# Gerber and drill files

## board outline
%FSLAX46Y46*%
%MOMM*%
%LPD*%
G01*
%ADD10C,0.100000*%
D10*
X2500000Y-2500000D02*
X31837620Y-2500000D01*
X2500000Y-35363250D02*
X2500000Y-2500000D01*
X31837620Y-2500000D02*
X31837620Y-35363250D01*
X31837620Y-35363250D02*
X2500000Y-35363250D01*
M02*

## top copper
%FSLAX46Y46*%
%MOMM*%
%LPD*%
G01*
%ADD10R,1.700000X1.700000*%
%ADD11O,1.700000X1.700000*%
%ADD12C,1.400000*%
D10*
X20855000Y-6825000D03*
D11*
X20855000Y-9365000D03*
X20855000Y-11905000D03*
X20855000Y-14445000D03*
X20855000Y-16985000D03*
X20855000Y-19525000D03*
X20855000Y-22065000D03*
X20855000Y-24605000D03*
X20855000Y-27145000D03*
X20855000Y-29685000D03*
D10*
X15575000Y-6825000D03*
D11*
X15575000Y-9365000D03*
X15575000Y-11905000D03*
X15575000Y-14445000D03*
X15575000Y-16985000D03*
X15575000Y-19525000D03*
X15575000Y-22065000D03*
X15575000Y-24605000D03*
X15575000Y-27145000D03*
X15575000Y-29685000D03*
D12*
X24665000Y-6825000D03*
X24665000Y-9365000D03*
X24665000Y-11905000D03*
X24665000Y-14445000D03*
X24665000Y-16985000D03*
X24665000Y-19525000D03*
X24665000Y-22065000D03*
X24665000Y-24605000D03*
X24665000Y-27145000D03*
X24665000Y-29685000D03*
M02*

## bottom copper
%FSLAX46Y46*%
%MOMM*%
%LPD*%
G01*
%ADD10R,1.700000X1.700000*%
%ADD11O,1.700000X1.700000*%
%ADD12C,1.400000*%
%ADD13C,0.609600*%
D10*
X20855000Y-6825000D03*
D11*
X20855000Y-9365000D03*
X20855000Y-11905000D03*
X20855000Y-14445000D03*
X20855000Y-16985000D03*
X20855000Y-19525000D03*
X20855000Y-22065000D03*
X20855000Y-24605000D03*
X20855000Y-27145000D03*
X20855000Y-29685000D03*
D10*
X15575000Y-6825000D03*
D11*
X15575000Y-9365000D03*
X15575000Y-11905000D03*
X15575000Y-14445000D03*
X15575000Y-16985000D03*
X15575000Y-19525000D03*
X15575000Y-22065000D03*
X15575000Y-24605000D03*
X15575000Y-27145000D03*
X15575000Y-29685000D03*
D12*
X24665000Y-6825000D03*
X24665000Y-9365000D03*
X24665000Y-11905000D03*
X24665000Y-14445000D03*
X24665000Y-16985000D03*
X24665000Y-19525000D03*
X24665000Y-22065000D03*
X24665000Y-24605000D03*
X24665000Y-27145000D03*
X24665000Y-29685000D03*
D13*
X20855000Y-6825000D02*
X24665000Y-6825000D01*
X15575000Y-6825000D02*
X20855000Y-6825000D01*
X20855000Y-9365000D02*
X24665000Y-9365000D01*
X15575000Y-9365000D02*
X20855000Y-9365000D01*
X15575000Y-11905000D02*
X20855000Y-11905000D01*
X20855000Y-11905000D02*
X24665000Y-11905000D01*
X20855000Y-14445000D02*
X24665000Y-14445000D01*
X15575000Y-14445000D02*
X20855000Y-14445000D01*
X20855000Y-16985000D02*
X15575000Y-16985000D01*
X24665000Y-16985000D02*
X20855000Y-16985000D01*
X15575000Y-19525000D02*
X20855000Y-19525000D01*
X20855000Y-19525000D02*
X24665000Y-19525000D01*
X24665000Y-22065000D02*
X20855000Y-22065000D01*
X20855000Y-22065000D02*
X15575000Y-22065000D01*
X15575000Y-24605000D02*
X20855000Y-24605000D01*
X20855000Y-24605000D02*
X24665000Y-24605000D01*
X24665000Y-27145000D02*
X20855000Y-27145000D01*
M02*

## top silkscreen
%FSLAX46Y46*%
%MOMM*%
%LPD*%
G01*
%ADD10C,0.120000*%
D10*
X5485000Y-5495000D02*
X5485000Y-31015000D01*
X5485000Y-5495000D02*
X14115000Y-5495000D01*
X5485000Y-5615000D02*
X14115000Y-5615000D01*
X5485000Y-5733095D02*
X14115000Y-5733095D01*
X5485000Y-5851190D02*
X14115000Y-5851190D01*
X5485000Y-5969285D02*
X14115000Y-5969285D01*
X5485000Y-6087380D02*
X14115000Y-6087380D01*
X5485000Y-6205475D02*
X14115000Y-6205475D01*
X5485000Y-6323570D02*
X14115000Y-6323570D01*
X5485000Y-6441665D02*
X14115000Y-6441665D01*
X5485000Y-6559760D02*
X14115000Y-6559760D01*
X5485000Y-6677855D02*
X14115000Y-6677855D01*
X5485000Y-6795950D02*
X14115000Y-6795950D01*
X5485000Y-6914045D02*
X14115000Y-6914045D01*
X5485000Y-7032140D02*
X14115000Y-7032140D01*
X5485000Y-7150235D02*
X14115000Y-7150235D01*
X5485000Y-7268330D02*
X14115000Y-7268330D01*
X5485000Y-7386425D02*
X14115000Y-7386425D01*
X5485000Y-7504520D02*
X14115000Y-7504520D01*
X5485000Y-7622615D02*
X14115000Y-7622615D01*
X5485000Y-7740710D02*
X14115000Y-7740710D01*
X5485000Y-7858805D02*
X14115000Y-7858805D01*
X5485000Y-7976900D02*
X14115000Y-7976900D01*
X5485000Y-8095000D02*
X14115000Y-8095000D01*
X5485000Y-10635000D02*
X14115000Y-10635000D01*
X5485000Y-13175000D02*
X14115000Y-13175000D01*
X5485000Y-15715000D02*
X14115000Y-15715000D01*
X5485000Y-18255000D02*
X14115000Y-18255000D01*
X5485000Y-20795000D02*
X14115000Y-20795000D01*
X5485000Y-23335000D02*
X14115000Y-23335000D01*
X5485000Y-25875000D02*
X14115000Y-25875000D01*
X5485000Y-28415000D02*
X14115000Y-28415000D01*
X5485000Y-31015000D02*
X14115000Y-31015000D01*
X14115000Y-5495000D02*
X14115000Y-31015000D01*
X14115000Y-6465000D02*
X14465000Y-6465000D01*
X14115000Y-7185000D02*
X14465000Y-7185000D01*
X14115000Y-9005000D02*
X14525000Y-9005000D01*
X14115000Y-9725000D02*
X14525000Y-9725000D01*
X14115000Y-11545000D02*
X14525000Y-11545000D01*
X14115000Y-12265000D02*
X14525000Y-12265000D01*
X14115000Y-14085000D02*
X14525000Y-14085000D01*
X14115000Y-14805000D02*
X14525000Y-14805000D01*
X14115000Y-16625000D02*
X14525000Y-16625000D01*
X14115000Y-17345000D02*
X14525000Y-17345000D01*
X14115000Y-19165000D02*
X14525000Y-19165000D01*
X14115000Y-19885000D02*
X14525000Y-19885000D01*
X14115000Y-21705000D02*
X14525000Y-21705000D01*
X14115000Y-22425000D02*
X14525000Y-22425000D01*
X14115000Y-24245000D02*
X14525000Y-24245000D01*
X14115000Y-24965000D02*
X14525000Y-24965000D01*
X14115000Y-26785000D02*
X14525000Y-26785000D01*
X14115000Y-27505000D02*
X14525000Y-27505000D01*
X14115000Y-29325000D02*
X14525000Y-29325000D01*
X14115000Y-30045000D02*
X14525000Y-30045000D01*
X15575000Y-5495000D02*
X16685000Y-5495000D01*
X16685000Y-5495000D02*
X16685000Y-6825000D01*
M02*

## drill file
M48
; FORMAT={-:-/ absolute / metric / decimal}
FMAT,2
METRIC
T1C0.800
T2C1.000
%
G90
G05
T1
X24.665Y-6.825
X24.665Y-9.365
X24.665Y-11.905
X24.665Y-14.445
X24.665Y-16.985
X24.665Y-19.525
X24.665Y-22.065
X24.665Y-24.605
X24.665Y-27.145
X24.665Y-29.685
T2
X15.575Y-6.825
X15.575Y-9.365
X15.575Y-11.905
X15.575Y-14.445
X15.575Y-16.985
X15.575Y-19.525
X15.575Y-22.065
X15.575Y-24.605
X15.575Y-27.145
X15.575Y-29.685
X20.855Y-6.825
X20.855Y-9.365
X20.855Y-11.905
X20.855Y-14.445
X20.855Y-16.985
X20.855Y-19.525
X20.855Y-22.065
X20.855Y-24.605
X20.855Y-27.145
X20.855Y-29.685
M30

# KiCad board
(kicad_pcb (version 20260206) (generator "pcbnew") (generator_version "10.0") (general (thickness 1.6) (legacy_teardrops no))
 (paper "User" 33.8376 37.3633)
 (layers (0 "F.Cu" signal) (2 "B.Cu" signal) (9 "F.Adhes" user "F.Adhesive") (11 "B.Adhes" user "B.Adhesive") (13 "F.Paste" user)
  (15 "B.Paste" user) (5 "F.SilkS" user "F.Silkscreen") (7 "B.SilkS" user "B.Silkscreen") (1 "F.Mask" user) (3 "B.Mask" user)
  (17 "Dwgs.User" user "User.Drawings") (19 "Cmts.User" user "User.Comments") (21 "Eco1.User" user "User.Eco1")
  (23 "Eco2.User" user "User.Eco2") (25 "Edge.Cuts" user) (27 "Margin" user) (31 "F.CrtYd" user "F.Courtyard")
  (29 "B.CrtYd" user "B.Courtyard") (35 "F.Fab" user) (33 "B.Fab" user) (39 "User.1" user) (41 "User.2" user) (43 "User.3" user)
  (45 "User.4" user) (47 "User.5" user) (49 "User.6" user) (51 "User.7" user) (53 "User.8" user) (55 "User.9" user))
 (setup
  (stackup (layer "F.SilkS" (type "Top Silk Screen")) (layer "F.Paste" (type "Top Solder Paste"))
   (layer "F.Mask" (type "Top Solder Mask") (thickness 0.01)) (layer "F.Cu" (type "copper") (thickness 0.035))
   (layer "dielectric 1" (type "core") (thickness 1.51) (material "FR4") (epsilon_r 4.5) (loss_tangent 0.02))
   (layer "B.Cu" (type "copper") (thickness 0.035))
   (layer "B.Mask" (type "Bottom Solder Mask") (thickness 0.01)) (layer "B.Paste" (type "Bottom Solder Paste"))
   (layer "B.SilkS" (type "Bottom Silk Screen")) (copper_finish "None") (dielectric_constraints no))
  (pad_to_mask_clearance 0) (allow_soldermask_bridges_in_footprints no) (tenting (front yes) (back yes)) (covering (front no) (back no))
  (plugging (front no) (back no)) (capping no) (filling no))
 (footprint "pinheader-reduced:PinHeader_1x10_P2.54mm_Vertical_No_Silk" (layer "F.Cu") (at 20.855 6.825)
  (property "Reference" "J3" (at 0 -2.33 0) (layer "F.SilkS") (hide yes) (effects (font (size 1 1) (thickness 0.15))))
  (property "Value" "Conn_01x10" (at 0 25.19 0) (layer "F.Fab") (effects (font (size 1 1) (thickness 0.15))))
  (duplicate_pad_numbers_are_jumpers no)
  (pad "1" thru_hole rect (at 0 0) (size 1.7 1.7) (drill 1) (layers "*.Cu" "*.Mask") (remove_unused_layers no) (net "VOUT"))
  (pad "2" thru_hole oval (at 0 2.54) (size 1.7 1.7) (drill 1) (layers "*.Cu" "*.Mask") (remove_unused_layers no) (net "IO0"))
  (pad "3" thru_hole oval (at 0 5.08) (size 1.7 1.7) (drill 1) (layers "*.Cu" "*.Mask") (remove_unused_layers no) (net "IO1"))
  (pad "4" thru_hole oval (at 0 7.62) (size 1.7 1.7) (drill 1) (layers "*.Cu" "*.Mask") (remove_unused_layers no) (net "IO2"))
  (pad "5" thru_hole oval (at 0 10.16) (size 1.7 1.7) (drill 1) (layers "*.Cu" "*.Mask") (remove_unused_layers no) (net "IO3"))
  (pad "6" thru_hole oval (at 0 12.7) (size 1.7 1.7) (drill 1) (layers "*.Cu" "*.Mask") (remove_unused_layers no) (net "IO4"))
  (pad "7" thru_hole oval (at 0 15.24) (size 1.7 1.7) (drill 1) (layers "*.Cu" "*.Mask") (remove_unused_layers no) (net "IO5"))
  (pad "8" thru_hole oval (at 0 17.78) (size 1.7 1.7) (drill 1) (layers "*.Cu" "*.Mask") (remove_unused_layers no) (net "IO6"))
  (pad "9" thru_hole oval (at 0 20.32) (size 1.7 1.7) (drill 1) (layers "*.Cu" "*.Mask") (remove_unused_layers no) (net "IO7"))
  (pad "10" thru_hole oval (at 0 22.86) (size 1.7 1.7) (drill 1) (layers "*.Cu" "*.Mask") (remove_unused_layers no) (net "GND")))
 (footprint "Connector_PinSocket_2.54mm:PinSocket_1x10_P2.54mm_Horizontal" (layer "F.Cu") (at 15.575 6.825)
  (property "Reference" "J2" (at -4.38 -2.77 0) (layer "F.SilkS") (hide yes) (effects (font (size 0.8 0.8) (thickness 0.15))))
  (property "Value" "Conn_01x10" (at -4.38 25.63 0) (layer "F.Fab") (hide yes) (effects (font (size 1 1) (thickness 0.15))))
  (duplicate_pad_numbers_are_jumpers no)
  (fp_line (start -10.09 -1.33) (end -10.09 24.19) (stroke (width 0.12) (type solid)) (layer "F.SilkS"))
  (fp_line (start -10.09 -1.33) (end -1.46 -1.33) (stroke (width 0.12) (type solid)) (layer "F.SilkS"))
  (fp_line (start -10.09 -1.21) (end -1.46 -1.21) (stroke (width 0.12) (type solid)) (layer "F.SilkS"))
  (fp_line (start -10.09 -1.091905) (end -1.46 -1.091905) (stroke (width 0.12) (type solid)) (layer "F.SilkS"))
  (fp_line (start -10.09 -0.97381) (end -1.46 -0.97381) (stroke (width 0.12) (type solid)) (layer "F.SilkS"))
  (fp_line (start -10.09 -0.855715) (end -1.46 -0.855715) (stroke (width 0.12) (type solid)) (layer "F.SilkS"))
  (fp_line (start -10.09 -0.73762) (end -1.46 -0.73762) (stroke (width 0.12) (type solid)) (layer "F.SilkS"))
  (fp_line (start -10.09 -0.619525) (end -1.46 -0.619525) (stroke (width 0.12) (type solid)) (layer "F.SilkS"))
  (fp_line (start -10.09 -0.50143) (end -1.46 -0.50143) (stroke (width 0.12) (type solid)) (layer "F.SilkS"))
  (fp_line (start -10.09 -0.383335) (end -1.46 -0.383335) (stroke (width 0.12) (type solid)) (layer "F.SilkS"))
  (fp_line (start -10.09 -0.26524) (end -1.46 -0.26524) (stroke (width 0.12) (type solid)) (layer "F.SilkS"))
  (fp_line (start -10.09 -0.147145) (end -1.46 -0.147145) (stroke (width 0.12) (type solid)) (layer "F.SilkS"))
  (fp_line (start -10.09 -0.02905) (end -1.46 -0.02905) (stroke (width 0.12) (type solid)) (layer "F.SilkS"))
  (fp_line (start -10.09 0.089045) (end -1.46 0.089045) (stroke (width 0.12) (type solid)) (layer "F.SilkS"))
  (fp_line (start -10.09 0.20714) (end -1.46 0.20714) (stroke (width 0.12) (type solid)) (layer "F.SilkS"))
  (fp_line (start -10.09 0.325235) (end -1.46 0.325235) (stroke (width 0.12) (type solid)) (layer "F.SilkS"))
  (fp_line (start -10.09 0.44333) (end -1.46 0.44333) (stroke (width 0.12) (type solid)) (layer "F.SilkS"))
  (fp_line (start -10.09 0.561425) (end -1.46 0.561425) (stroke (width 0.12) (type solid)) (layer "F.SilkS"))
  (fp_line (start -10.09 0.67952) (end -1.46 0.67952) (stroke (width 0.12) (type solid)) (layer "F.SilkS"))
  (fp_line (start -10.09 0.797615) (end -1.46 0.797615) (stroke (width 0.12) (type solid)) (layer "F.SilkS"))
  (fp_line (start -10.09 0.91571) (end -1.46 0.91571) (stroke (width 0.12) (type solid)) (layer "F.SilkS"))
  (fp_line (start -10.09 1.033805) (end -1.46 1.033805) (stroke (width 0.12) (type solid)) (layer "F.SilkS"))
  (fp_line (start -10.09 1.1519) (end -1.46 1.1519) (stroke (width 0.12) (type solid)) (layer "F.SilkS"))
  (fp_line (start -10.09 1.27) (end -1.46 1.27) (stroke (width 0.12) (type solid)) (layer "F.SilkS"))
  (fp_line (start -10.09 3.81) (end -1.46 3.81) (stroke (width 0.12) (type solid)) (layer "F.SilkS"))
  (fp_line (start -10.09 6.35) (end -1.46 6.35) (stroke (width 0.12) (type solid)) (layer "F.SilkS"))
  (fp_line (start -10.09 8.89) (end -1.46 8.89) (stroke (width 0.12) (type solid)) (layer "F.SilkS"))
  (fp_line (start -10.09 11.43) (end -1.46 11.43) (stroke (width 0.12) (type solid)) (layer "F.SilkS"))
  (fp_line (start -10.09 13.97) (end -1.46 13.97) (stroke (width 0.12) (type solid)) (layer "F.SilkS"))
  (fp_line (start -10.09 16.51) (end -1.46 16.51) (stroke (width 0.12) (type solid)) (layer "F.SilkS"))
  (fp_line (start -10.09 19.05) (end -1.46 19.05) (stroke (width 0.12) (type solid)) (layer "F.SilkS"))
  (fp_line (start -10.09 21.59) (end -1.46 21.59) (stroke (width 0.12) (type solid)) (layer "F.SilkS"))
  (fp_line (start -10.09 24.19) (end -1.46 24.19) (stroke (width 0.12) (type solid)) (layer "F.SilkS"))
  (fp_line (start -1.46 -1.33) (end -1.46 24.19) (stroke (width 0.12) (type solid)) (layer "F.SilkS"))
  (fp_line (start -1.46 -0.36) (end -1.11 -0.36) (stroke (width 0.12) (type solid)) (layer "F.SilkS"))
  (fp_line (start -1.46 0.36) (end -1.11 0.36) (stroke (width 0.12) (type solid)) (layer "F.SilkS"))
  (fp_line (start -1.46 2.18) (end -1.05 2.18) (stroke (width 0.12) (type solid)) (layer "F.SilkS"))
  (fp_line (start -1.46 2.9) (end -1.05 2.9) (stroke (width 0.12) (type solid)) (layer "F.SilkS"))
  (fp_line (start -1.46 4.72) (end -1.05 4.72) (stroke (width 0.12) (type solid)) (layer "F.SilkS"))
  (fp_line (start -1.46 5.44) (end -1.05 5.44) (stroke (width 0.12) (type solid)) (layer "F.SilkS"))
  (fp_line (start -1.46 7.26) (end -1.05 7.26) (stroke (width 0.12) (type solid)) (layer "F.SilkS"))
  (fp_line (start -1.46 7.98) (end -1.05 7.98) (stroke (width 0.12) (type solid)) (layer "F.SilkS"))
  (fp_line (start -1.46 9.8) (end -1.05 9.8) (stroke (width 0.12) (type solid)) (layer "F.SilkS"))
  (fp_line (start -1.46 10.52) (end -1.05 10.52) (stroke (width 0.12) (type solid)) (layer "F.SilkS"))
  (fp_line (start -1.46 12.34) (end -1.05 12.34) (stroke (width 0.12) (type solid)) (layer "F.SilkS"))
  (fp_line (start -1.46 13.06) (end -1.05 13.06) (stroke (width 0.12) (type solid)) (layer "F.SilkS"))
  (fp_line (start -1.46 14.88) (end -1.05 14.88) (stroke (width 0.12) (type solid)) (layer "F.SilkS"))
  (fp_line (start -1.46 15.6) (end -1.05 15.6) (stroke (width 0.12) (type solid)) (layer "F.SilkS"))
  (fp_line (start -1.46 17.42) (end -1.05 17.42) (stroke (width 0.12) (type solid)) (layer "F.SilkS"))
  (fp_line (start -1.46 18.14) (end -1.05 18.14) (stroke (width 0.12) (type solid)) (layer "F.SilkS"))
  (fp_line (start -1.46 19.96) (end -1.05 19.96) (stroke (width 0.12) (type solid)) (layer "F.SilkS"))
  (fp_line (start -1.46 20.68) (end -1.05 20.68) (stroke (width 0.12) (type solid)) (layer "F.SilkS"))
  (fp_line (start -1.46 22.5) (end -1.05 22.5) (stroke (width 0.12) (type solid)) (layer "F.SilkS"))
  (fp_line (start -1.46 23.22) (end -1.05 23.22) (stroke (width 0.12) (type solid)) (layer "F.SilkS"))
  (fp_line (start 0 -1.33) (end 1.11 -1.33) (stroke (width 0.12) (type solid)) (layer "F.SilkS"))
  (fp_line (start 1.11 -1.33) (end 1.11 0) (stroke (width 0.12) (type solid)) (layer "F.SilkS"))
  (pad "1" thru_hole rect (at 0 0) (size 1.7 1.7) (drill 1) (layers "*.Cu" "*.Mask") (remove_unused_layers no) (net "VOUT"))
  (pad "2" thru_hole oval (at 0 2.54) (size 1.7 1.7) (drill 1) (layers "*.Cu" "*.Mask") (remove_unused_layers no) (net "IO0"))
  (pad "3" thru_hole oval (at 0 5.08) (size 1.7 1.7) (drill 1) (layers "*.Cu" "*.Mask") (remove_unused_layers no) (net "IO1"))
  (pad "4" thru_hole oval (at 0 7.62) (size 1.7 1.7) (drill 1) (layers "*.Cu" "*.Mask") (remove_unused_layers no) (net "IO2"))
  (pad "5" thru_hole oval (at 0 10.16) (size 1.7 1.7) (drill 1) (layers "*.Cu" "*.Mask") (remove_unused_layers no) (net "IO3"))
  (pad "6" thru_hole oval (at 0 12.7) (size 1.7 1.7) (drill 1) (layers "*.Cu" "*.Mask") (remove_unused_layers no) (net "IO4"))
  (pad "7" thru_hole oval (at 0 15.24) (size 1.7 1.7) (drill 1) (layers "*.Cu" "*.Mask") (remove_unused_layers no) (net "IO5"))
  (pad "8" thru_hole oval (at 0 17.78) (size 1.7 1.7) (drill 1) (layers "*.Cu" "*.Mask") (remove_unused_layers no) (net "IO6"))
  (pad "9" thru_hole oval (at 0 20.32) (size 1.7 1.7) (drill 1) (layers "*.Cu" "*.Mask") (remove_unused_layers no) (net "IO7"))
  (pad "10" thru_hole oval (at 0 22.86) (size 1.7 1.7) (drill 1) (layers "*.Cu" "*.Mask") (remove_unused_layers no) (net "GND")))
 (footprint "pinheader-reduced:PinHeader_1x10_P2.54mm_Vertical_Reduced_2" (layer "F.Cu") (at 24.665 6.825)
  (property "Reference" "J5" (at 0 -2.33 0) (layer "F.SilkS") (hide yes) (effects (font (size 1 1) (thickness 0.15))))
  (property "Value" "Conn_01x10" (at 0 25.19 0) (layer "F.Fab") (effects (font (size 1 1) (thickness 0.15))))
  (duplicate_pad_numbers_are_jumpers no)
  (pad "1" thru_hole circle (at 0 0) (size 1.4 1.4) (drill 0.8) (layers "*.Cu" "*.Mask") (remove_unused_layers no) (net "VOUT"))
  (pad "2" thru_hole circle (at 0 2.54) (size 1.4 1.4) (drill 0.8) (layers "*.Cu" "*.Mask") (remove_unused_layers no) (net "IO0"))
  (pad "3" thru_hole circle (at 0 5.08) (size 1.4 1.4) (drill 0.8) (layers "*.Cu" "*.Mask") (remove_unused_layers no) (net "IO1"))
  (pad "4" thru_hole circle (at 0 7.62) (size 1.4 1.4) (drill 0.8) (layers "*.Cu" "*.Mask") (remove_unused_layers no) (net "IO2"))
  (pad "5" thru_hole circle (at 0 10.16) (size 1.4 1.4) (drill 0.8) (layers "*.Cu" "*.Mask") (remove_unused_layers no) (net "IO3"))
  (pad "6" thru_hole circle (at 0 12.7) (size 1.4 1.4) (drill 0.8) (layers "*.Cu" "*.Mask") (remove_unused_layers no) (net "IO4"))
  (pad "7" thru_hole circle (at 0 15.24) (size 1.4 1.4) (drill 0.8) (layers "*.Cu" "*.Mask") (remove_unused_layers no) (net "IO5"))
  (pad "8" thru_hole circle (at 0 17.78) (size 1.4 1.4) (drill 0.8) (layers "*.Cu" "*.Mask") (remove_unused_layers no) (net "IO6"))
  (pad "9" thru_hole circle (at 0 20.32) (size 1.4 1.4) (drill 0.8) (layers "*.Cu" "*.Mask") (remove_unused_layers no) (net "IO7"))
  (pad "10" thru_hole circle (at 0 22.86) (size 1.4 1.4) (drill 0.8) (layers "*.Cu" "*.Mask") (remove_unused_layers no) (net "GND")))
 (gr_line (start 2.5 2.5) (end 31.83762 2.5) (stroke (width 0.1) (type default)) (layer "Edge.Cuts"))
 (gr_line (start 2.5 35.36325) (end 2.5 2.5) (stroke (width 0.1) (type default)) (layer "Edge.Cuts"))
 (gr_line (start 31.83762 2.5) (end 31.83762 35.36325) (stroke (width 0.1) (type default)) (layer "Edge.Cuts"))
 (gr_line (start 31.83762 35.36325) (end 2.5 35.36325) (stroke (width 0.1) (type default)) (layer "Edge.Cuts"))
 (segment (start 20.855 6.825) (end 24.665 6.825) (width 0.6096) (layer "B.Cu") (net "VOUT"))
 (segment (start 15.575 6.825) (end 20.855 6.825) (width 0.6096) (layer "B.Cu") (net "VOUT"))
 (segment (start 20.855 9.365) (end 24.665 9.365) (width 0.6096) (layer "B.Cu") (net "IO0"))
 (segment (start 15.575 9.365) (end 20.855 9.365) (width 0.6096) (layer "B.Cu") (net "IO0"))
 (segment (start 15.575 11.905) (end 20.855 11.905) (width 0.6096) (layer "B.Cu") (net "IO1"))
 (segment (start 20.855 11.905) (end 24.665 11.905) (width 0.6096) (layer "B.Cu") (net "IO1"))
 (segment (start 20.855 14.445) (end 24.665 14.445) (width 0.6096) (layer "B.Cu") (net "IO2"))
 (segment (start 15.575 14.445) (end 20.855 14.445) (width 0.6096) (layer "B.Cu") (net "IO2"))
 (segment (start 20.855 16.985) (end 15.575 16.985) (width 0.6096) (layer "B.Cu") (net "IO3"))
 (segment (start 24.665 16.985) (end 20.855 16.985) (width 0.6096) (layer "B.Cu") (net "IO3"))
 (segment (start 15.575 19.525) (end 20.855 19.525) (width 0.6096) (layer "B.Cu") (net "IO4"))
 (segment (start 20.855 19.525) (end 24.665 19.525) (width 0.6096) (layer "B.Cu") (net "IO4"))
 (segment (start 24.665 22.065) (end 20.855 22.065) (width 0.6096) (layer "B.Cu") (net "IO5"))
 (segment (start 20.855 22.065) (end 15.575 22.065) (width 0.6096) (layer "B.Cu") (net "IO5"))
 (segment (start 15.575 24.605) (end 20.855 24.605) (width 0.6096) (layer "B.Cu") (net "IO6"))
 (segment (start 20.855 24.605) (end 24.665 24.605) (width 0.6096) (layer "B.Cu") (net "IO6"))
 (segment (start 24.665 27.145) (end 20.855 27.145) (width 0.6096) (layer "B.Cu") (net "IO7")))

